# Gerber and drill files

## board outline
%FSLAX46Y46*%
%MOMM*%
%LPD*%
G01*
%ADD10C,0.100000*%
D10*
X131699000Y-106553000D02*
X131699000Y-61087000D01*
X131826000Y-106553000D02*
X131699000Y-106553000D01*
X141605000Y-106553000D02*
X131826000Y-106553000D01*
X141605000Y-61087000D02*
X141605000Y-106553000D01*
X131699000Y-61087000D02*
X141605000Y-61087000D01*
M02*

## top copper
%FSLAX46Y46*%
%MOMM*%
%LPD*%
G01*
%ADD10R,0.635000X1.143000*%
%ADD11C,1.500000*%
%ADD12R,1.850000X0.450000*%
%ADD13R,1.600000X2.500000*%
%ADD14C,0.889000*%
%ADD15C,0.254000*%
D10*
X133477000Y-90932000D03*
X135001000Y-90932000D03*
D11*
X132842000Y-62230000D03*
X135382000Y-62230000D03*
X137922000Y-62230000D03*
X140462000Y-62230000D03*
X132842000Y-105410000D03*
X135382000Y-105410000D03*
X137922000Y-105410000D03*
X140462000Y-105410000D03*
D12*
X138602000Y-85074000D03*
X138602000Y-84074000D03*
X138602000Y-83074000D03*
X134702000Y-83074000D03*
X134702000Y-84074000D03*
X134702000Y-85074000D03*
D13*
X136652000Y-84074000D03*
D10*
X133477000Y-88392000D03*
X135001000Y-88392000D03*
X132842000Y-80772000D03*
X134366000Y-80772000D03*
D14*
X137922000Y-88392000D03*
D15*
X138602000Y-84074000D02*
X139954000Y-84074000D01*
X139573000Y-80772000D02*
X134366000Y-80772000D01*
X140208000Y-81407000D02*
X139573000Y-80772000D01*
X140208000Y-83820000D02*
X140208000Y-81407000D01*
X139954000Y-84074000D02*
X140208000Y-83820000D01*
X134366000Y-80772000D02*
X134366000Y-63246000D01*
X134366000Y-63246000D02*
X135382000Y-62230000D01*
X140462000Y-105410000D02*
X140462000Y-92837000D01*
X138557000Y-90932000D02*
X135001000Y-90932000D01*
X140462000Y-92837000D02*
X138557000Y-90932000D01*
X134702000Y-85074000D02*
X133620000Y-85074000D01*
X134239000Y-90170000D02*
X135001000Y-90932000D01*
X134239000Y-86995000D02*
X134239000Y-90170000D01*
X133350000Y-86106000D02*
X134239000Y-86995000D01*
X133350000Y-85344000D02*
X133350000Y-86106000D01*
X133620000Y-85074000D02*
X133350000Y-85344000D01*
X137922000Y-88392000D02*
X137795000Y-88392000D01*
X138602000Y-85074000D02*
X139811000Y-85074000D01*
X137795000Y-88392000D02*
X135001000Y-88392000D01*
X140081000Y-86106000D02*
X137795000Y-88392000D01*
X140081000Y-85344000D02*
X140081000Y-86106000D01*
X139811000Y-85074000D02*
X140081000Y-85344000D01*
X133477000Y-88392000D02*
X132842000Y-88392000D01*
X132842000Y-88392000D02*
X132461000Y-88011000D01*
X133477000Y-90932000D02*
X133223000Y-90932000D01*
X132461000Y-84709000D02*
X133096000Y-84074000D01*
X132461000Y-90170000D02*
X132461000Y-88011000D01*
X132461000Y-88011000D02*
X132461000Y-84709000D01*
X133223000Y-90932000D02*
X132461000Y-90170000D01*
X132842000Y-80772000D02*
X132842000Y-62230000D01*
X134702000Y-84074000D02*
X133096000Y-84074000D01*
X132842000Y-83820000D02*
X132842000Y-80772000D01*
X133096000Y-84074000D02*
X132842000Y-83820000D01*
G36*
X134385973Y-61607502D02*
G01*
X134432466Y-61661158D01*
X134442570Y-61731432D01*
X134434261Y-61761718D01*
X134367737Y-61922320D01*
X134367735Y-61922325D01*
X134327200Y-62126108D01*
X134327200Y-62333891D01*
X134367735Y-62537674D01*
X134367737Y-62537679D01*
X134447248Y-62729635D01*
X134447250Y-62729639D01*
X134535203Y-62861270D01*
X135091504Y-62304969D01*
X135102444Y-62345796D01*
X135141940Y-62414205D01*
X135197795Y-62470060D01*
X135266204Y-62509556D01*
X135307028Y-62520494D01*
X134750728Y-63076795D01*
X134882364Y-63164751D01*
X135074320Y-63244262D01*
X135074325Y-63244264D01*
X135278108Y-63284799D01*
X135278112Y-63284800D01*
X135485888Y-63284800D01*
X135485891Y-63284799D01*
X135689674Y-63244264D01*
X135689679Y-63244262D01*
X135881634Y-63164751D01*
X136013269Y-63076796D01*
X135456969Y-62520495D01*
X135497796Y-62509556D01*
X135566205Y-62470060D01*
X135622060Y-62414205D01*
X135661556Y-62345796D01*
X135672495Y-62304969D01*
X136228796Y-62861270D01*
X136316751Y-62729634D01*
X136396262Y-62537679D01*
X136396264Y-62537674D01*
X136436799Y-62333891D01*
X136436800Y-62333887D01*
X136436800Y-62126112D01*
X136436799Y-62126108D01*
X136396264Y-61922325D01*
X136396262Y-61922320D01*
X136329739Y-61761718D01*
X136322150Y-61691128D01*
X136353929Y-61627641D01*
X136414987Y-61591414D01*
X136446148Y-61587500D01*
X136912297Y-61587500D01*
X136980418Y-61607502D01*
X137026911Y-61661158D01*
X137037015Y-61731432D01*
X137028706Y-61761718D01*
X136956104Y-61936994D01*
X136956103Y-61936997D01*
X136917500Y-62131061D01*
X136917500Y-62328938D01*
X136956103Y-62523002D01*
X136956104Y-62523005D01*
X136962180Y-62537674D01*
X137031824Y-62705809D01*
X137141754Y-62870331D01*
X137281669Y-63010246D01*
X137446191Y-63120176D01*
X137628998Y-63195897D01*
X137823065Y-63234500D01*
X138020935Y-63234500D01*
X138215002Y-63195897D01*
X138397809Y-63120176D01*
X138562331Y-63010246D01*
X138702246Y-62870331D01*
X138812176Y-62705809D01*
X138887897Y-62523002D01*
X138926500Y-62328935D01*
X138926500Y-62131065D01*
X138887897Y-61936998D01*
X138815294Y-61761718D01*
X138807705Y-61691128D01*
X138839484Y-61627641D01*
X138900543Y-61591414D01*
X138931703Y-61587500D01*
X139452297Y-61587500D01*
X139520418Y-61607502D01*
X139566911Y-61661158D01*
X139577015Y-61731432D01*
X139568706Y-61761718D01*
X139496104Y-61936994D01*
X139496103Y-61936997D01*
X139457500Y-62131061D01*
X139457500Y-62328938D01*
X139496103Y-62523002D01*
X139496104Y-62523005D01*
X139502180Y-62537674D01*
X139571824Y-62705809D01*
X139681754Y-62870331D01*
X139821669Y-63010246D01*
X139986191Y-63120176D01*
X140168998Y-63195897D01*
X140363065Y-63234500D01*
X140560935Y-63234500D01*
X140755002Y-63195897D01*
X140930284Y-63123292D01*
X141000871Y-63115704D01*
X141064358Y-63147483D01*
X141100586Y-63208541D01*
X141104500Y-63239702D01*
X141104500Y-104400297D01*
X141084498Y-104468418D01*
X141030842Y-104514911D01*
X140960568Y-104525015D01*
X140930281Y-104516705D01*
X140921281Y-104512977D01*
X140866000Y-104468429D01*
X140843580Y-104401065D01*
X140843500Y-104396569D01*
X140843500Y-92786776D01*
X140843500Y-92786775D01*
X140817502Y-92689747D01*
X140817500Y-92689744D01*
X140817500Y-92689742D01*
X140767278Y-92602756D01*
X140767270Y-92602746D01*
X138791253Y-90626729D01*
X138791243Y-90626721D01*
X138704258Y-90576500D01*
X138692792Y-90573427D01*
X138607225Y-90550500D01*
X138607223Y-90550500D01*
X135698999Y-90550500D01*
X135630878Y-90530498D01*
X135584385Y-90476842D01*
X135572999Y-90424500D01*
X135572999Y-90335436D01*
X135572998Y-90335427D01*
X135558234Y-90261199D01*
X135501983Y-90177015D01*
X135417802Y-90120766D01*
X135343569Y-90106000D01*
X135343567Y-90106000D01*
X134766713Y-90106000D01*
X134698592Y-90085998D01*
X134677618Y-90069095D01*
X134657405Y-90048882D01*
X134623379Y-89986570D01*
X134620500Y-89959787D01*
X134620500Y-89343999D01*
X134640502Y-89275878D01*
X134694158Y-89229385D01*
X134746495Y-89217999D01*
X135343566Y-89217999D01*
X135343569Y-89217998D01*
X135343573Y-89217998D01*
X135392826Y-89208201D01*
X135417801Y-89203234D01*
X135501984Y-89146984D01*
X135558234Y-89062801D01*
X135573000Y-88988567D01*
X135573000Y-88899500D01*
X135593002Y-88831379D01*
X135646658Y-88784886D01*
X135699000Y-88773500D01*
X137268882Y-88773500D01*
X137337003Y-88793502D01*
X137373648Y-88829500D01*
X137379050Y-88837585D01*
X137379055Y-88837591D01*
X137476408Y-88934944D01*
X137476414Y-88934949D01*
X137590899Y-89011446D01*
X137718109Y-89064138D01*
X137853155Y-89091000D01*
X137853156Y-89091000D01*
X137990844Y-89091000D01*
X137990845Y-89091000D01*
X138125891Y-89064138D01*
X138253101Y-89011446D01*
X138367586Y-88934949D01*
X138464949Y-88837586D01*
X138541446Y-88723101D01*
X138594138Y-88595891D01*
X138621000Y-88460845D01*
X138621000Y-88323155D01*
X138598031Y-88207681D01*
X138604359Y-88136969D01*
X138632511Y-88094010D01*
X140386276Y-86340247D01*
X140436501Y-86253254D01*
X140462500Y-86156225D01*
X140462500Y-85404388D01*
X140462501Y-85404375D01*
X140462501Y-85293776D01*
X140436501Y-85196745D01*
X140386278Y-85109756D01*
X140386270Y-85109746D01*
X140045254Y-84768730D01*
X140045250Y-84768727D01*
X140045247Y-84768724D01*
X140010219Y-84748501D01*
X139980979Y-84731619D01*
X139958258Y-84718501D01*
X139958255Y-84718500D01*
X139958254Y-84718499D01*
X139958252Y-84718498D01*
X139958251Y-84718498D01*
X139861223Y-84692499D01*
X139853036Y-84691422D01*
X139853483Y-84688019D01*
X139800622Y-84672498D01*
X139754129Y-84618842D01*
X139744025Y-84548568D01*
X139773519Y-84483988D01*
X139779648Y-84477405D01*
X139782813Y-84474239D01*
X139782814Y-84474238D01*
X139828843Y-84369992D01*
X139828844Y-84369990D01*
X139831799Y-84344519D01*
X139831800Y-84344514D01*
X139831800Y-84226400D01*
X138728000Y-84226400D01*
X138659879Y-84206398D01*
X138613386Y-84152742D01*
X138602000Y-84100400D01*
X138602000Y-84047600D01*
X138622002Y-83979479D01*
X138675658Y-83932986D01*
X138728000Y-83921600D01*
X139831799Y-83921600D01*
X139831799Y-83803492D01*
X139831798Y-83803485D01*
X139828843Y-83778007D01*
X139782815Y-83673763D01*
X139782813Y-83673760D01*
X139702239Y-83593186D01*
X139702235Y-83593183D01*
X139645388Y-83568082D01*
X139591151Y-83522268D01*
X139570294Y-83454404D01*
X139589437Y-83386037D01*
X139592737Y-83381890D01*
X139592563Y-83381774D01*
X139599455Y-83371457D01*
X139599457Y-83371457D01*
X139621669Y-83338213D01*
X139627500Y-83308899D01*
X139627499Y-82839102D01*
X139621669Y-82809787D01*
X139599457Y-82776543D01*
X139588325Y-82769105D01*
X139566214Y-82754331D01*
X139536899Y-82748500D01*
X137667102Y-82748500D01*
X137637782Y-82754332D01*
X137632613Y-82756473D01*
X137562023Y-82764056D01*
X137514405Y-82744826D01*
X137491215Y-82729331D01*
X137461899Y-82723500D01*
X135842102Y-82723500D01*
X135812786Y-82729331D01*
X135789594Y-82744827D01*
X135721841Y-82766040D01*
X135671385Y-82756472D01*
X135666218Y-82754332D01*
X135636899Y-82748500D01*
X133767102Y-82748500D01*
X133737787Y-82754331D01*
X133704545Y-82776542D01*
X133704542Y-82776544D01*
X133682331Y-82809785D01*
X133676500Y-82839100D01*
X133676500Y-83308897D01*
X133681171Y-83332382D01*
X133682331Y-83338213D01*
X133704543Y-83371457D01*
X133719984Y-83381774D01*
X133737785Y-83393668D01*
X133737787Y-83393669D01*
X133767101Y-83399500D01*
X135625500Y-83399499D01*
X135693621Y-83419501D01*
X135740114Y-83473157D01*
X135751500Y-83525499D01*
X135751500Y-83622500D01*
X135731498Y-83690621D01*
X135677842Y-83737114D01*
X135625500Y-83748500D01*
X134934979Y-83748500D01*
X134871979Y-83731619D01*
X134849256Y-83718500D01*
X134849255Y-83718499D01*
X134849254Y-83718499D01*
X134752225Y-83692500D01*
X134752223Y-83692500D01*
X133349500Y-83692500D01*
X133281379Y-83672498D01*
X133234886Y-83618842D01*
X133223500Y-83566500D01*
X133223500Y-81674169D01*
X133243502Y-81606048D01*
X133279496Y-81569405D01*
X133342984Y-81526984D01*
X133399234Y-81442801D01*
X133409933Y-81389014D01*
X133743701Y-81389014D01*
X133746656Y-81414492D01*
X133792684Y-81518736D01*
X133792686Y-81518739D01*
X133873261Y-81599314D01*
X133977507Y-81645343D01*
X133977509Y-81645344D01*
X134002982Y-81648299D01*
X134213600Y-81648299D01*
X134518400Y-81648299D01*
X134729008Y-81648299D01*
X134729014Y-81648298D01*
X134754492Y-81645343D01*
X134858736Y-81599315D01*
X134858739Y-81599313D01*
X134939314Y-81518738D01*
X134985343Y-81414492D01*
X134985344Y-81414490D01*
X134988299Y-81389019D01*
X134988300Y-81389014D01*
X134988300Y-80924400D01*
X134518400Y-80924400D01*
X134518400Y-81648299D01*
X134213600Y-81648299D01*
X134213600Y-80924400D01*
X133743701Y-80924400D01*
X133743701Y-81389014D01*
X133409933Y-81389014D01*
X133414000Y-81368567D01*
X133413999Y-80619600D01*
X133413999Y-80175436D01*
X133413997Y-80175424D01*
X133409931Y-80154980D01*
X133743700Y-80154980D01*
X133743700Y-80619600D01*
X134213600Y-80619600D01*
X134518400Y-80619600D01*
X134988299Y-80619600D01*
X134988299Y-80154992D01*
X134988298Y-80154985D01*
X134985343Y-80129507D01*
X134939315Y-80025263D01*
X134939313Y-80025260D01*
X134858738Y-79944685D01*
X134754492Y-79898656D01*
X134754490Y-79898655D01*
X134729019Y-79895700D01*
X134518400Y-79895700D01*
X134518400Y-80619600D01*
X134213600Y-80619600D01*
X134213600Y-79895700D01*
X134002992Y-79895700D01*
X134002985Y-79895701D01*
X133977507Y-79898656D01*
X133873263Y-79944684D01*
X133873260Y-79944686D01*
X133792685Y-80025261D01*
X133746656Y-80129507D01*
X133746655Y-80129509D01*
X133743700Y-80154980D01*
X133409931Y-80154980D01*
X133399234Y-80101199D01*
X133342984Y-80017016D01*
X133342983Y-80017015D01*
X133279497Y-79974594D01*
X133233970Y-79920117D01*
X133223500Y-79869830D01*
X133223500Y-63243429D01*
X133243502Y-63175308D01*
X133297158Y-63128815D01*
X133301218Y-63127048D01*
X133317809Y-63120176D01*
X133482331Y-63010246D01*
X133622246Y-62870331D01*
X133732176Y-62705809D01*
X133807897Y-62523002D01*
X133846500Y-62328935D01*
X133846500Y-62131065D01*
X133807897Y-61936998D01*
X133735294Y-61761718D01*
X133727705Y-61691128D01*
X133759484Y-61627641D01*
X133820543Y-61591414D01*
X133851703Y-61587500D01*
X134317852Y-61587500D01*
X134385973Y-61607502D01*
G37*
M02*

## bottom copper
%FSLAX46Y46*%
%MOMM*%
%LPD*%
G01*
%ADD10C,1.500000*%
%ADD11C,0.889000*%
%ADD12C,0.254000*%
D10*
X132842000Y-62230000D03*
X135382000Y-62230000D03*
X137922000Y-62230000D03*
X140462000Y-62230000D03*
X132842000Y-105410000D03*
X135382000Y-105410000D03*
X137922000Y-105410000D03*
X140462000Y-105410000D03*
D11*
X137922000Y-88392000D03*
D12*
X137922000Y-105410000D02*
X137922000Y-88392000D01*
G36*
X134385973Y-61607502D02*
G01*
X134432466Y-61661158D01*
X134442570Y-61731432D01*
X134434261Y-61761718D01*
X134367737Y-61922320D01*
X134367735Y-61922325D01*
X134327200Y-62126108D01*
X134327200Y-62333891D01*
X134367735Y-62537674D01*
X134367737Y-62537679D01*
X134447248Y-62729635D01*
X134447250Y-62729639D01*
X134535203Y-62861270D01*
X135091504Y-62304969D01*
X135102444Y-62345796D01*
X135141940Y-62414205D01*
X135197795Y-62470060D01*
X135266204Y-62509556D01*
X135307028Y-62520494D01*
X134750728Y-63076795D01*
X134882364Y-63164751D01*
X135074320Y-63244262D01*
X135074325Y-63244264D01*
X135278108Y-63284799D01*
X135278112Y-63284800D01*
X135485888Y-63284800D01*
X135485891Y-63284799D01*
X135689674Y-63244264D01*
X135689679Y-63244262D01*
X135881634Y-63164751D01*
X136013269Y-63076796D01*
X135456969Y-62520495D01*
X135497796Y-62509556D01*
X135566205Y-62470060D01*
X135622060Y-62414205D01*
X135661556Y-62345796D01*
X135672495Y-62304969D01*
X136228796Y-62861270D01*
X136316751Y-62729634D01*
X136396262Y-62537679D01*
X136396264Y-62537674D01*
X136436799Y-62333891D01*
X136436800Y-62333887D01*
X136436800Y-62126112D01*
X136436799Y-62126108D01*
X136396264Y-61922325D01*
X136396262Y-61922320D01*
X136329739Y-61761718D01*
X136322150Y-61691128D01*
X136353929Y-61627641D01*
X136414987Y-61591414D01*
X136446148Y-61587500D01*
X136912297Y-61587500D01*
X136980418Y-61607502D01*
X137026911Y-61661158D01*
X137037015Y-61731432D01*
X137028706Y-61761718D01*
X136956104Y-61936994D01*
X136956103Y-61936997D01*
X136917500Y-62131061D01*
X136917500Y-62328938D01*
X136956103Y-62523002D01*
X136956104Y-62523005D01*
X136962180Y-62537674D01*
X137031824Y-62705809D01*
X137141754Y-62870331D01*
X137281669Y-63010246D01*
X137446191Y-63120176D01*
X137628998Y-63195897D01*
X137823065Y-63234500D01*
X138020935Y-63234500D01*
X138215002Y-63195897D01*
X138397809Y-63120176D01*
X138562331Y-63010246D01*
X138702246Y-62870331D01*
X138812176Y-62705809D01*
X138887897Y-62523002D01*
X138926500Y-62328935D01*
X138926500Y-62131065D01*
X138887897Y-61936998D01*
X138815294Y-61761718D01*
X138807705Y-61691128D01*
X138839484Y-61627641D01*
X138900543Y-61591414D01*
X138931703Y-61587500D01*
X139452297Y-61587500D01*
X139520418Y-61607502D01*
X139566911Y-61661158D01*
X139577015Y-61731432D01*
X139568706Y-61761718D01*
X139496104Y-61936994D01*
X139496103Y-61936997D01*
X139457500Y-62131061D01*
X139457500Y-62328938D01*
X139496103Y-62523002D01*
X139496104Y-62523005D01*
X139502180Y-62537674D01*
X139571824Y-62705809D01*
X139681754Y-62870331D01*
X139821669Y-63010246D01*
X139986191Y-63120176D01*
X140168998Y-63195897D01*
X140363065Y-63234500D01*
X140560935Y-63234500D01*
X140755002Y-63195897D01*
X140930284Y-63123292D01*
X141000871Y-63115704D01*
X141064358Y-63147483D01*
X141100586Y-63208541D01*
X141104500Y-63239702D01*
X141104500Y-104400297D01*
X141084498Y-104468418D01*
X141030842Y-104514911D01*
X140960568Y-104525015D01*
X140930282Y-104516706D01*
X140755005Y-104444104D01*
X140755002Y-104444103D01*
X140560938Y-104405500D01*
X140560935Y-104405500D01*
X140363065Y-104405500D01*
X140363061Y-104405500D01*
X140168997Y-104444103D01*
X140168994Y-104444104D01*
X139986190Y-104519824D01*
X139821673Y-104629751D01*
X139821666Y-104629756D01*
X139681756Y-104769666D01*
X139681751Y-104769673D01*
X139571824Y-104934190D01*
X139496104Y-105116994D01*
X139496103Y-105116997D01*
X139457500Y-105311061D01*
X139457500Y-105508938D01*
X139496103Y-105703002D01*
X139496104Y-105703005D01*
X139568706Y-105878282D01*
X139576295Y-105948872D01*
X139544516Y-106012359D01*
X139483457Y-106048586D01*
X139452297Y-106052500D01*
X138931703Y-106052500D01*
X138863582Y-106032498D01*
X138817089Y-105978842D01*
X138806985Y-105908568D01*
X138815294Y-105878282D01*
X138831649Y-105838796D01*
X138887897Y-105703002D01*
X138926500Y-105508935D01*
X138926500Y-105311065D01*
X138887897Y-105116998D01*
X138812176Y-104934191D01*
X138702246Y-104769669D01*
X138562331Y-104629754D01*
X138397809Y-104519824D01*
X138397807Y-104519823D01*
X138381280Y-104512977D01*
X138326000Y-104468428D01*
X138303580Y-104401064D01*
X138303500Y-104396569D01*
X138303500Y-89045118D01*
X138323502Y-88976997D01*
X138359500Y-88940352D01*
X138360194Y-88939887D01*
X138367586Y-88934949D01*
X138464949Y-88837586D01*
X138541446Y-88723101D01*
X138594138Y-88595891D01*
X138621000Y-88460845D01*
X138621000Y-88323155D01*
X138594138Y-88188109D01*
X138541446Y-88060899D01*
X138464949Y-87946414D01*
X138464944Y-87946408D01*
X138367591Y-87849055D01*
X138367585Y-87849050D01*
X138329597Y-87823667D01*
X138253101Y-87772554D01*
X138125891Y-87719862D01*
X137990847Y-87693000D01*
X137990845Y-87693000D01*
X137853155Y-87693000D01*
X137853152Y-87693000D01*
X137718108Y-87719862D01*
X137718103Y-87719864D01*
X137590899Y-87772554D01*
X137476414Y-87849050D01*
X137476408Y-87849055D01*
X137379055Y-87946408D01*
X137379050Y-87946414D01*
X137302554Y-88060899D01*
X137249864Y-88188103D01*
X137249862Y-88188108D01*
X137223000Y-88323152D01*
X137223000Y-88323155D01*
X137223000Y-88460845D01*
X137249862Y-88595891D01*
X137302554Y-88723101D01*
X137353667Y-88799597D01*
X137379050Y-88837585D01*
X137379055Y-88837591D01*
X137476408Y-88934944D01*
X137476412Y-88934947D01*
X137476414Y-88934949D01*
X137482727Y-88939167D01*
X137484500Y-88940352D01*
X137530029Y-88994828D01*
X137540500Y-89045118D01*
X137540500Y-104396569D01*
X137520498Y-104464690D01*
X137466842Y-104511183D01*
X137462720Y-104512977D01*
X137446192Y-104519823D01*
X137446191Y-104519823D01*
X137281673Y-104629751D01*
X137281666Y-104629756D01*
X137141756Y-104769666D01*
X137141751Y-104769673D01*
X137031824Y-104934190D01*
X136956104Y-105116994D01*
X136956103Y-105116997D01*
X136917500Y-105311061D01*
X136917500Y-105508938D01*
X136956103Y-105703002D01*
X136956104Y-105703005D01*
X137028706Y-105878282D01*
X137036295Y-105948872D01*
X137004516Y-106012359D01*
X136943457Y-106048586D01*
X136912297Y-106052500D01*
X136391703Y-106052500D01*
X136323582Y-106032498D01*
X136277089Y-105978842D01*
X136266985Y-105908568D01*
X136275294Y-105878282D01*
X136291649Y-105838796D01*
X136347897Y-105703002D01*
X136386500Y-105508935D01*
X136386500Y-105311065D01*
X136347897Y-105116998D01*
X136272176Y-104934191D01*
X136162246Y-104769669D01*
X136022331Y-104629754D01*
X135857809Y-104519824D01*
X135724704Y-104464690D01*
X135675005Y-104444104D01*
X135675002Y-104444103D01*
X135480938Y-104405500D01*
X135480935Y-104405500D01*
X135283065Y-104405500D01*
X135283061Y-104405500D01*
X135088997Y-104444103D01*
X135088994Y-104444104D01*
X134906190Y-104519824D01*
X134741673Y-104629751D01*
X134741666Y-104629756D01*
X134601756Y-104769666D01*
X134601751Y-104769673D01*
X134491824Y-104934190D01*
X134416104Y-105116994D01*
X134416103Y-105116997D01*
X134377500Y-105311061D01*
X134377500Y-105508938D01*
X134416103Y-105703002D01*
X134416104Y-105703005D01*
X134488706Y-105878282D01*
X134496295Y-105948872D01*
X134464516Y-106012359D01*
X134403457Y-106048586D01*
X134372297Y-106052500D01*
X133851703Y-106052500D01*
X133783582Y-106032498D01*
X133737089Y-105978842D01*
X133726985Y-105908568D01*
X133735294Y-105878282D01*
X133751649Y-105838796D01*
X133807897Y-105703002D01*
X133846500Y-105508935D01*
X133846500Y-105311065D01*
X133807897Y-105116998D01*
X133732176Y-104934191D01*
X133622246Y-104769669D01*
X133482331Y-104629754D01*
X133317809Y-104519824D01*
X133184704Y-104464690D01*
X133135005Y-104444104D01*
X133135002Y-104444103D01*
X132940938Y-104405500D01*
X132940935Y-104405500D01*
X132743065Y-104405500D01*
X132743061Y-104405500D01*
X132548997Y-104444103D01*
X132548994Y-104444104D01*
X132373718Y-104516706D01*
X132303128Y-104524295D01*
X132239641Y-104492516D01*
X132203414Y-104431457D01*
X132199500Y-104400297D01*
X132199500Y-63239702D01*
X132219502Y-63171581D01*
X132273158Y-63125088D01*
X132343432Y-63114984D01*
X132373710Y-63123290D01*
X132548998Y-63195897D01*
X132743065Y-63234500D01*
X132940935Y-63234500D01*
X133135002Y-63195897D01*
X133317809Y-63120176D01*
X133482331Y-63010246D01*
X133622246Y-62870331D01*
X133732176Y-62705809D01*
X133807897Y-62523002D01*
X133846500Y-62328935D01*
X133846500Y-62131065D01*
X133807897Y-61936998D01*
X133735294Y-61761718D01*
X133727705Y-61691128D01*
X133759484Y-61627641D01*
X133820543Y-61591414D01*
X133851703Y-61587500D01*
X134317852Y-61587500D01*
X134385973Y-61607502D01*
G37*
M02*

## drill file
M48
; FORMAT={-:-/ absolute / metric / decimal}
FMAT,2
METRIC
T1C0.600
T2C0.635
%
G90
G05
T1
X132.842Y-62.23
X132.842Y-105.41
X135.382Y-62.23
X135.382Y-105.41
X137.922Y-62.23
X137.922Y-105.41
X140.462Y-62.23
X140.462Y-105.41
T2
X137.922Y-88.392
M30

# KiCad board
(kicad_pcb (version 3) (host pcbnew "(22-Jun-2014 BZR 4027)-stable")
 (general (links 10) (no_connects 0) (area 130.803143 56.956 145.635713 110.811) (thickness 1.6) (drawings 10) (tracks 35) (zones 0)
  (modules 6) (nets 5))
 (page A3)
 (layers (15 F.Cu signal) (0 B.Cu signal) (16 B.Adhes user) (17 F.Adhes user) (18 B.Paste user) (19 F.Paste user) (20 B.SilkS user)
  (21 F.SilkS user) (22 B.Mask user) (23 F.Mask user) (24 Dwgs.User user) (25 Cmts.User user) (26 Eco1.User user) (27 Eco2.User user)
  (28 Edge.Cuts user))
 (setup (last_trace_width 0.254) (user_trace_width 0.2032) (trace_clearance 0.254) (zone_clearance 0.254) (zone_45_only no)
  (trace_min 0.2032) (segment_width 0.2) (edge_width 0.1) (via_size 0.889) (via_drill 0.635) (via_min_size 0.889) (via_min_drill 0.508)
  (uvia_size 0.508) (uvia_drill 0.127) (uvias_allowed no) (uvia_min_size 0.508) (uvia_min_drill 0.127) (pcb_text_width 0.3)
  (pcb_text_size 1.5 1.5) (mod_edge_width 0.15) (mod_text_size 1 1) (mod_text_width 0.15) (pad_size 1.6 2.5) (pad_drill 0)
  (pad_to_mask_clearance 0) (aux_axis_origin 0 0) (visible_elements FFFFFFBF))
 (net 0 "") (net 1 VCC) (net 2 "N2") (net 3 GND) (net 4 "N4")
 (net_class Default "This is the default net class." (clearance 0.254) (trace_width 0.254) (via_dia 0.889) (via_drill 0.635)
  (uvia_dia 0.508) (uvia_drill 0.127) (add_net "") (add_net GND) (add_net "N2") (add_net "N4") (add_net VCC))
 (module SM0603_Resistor (layer F.Cu) (at 134.239 90.932)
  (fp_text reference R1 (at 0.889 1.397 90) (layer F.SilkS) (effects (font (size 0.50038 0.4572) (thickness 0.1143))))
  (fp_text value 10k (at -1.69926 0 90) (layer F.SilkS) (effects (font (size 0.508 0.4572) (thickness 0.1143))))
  (pad 1 smd rect (at -0.762 0) (size 0.635 1.143) (layers F.Cu F.Paste F.Mask) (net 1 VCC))
  (pad 2 smd rect (at 0.762 0) (size 0.635 1.143) (layers F.Cu F.Paste F.Mask) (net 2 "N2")))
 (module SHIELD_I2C (layer F.Cu) (at 136.652 83.82)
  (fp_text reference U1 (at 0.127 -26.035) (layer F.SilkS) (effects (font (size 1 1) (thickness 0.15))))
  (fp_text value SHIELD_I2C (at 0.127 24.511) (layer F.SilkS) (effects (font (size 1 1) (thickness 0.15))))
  (pad 1 thru_hole circle (at -3.81 -21.59) (size 1.5 1.5) (drill 0.6) (layers *.Cu *.Mask F.SilkS) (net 1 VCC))
  (pad 2 thru_hole circle (at -1.27 -21.59) (size 1.5 1.5) (drill 0.6) (layers *.Cu *.Mask F.SilkS) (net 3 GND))
  (pad 3 thru_hole circle (at 1.27 -21.59) (size 1.5 1.5) (drill 0.6) (layers *.Cu *.Mask F.SilkS))
  (pad 4 thru_hole circle (at 3.81 -21.59) (size 1.5 1.5) (drill 0.6) (layers *.Cu *.Mask F.SilkS))
  (pad 5 thru_hole circle (at -3.81 21.59) (size 1.5 1.5) (drill 0.6) (layers *.Cu *.Mask F.SilkS))
  (pad 6 thru_hole circle (at -1.27 21.59) (size 1.5 1.5) (drill 0.6) (layers *.Cu *.Mask F.SilkS))
  (pad 7 thru_hole circle (at 1.27 21.59) (size 1.5 1.5) (drill 0.6) (layers *.Cu *.Mask F.SilkS) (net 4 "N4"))
  (pad 8 thru_hole circle (at 3.81 21.59) (size 1.5 1.5) (drill 0.6) (layers *.Cu *.Mask F.SilkS) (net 2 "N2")))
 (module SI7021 (layer F.Cu) (at 136.652 84.074 180) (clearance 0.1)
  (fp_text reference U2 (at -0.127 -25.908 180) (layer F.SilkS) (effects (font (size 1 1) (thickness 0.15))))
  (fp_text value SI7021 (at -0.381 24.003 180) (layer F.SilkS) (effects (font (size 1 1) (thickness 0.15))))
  (pad 1 smd rect (at -1.95 -1 180) (size 1.85 0.45) (layers F.Cu F.Paste F.Mask) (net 4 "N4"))
  (pad 2 smd rect (at -1.95 0 180) (size 1.85 0.45) (layers F.Cu F.Paste F.Mask) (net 3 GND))
  (pad 3 smd rect (at -1.95 1 180) (size 1.85 0.45) (layers F.Cu F.Paste F.Mask))
  (pad 4 smd rect (at 1.95 1 180) (size 1.85 0.45) (layers F.Cu F.Paste F.Mask))
  (pad 5 smd rect (at 1.95 0 180) (size 1.85 0.45) (layers F.Cu F.Paste F.Mask) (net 1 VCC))
  (pad 6 smd rect (at 1.95 -1 180) (size 1.85 0.45) (layers F.Cu F.Paste F.Mask) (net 2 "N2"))
  (pad 7 smd rect (at 0 0 180) (size 1.6 2.5) (layers F.Cu F.Paste F.Mask)))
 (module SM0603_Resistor (layer F.Cu) (at 134.239 88.392)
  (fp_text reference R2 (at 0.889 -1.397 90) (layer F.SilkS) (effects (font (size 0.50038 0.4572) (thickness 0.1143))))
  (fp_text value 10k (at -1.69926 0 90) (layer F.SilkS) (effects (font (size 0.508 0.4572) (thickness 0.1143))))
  (pad 1 smd rect (at -0.762 0) (size 0.635 1.143) (layers F.Cu F.Paste F.Mask) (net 1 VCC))
  (pad 2 smd rect (at 0.762 0) (size 0.635 1.143) (layers F.Cu F.Paste F.Mask) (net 4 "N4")))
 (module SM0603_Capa (layer F.Cu) (at 133.604 80.772)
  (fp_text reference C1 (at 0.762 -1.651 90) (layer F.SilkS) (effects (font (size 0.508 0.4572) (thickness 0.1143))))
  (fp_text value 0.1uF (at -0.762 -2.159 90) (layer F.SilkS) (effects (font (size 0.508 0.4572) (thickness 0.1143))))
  (pad 1 smd rect (at -0.762 0) (size 0.635 1.143) (layers F.Cu F.Paste F.Mask) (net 1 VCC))
  (pad 2 smd rect (at 0.762 0) (size 0.635 1.143) (layers F.Cu F.Paste F.Mask) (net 3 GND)))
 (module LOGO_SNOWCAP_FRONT (layer F.Cu) (at 138.811 71.501 90)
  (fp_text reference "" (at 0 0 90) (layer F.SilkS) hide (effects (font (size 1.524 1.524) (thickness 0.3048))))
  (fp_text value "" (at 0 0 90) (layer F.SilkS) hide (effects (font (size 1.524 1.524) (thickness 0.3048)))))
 (gr_line (start 131.699 106.553) (end 131.699 61.087) (angle 90) (layer Edge.Cuts) (width 0.1))
 (gr_line (start 131.826 106.553) (end 131.699 106.553) (angle 90) (layer Edge.Cuts) (width 0.1))
 (gr_line (start 141.605 106.553) (end 131.826 106.553) (angle 90) (layer Edge.Cuts) (width 0.1))
 (gr_line (start 141.605 61.087) (end 141.605 106.553) (angle 90) (layer Edge.Cuts) (width 0.1))
 (gr_line (start 131.699 61.087) (end 141.605 61.087) (angle 90) (layer Edge.Cuts) (width 0.1))
 (segment (start 138.602 84.074) (end 139.954 84.074) (width 0.254) (layer F.Cu) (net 3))
 (segment (start 139.573 80.772) (end 134.366 80.772) (width 0.254) (layer F.Cu) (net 3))
 (segment (start 140.208 81.407) (end 139.573 80.772) (width 0.254) (layer F.Cu) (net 3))
 (segment (start 140.208 83.82) (end 140.208 81.407) (width 0.254) (layer F.Cu) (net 3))
 (segment (start 139.954 84.074) (end 140.208 83.82) (width 0.254) (layer F.Cu) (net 3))
 (segment (start 134.366 80.772) (end 134.366 63.246) (width 0.254) (layer F.Cu) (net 3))
 (segment (start 134.366 63.246) (end 135.382 62.23) (width 0.254) (layer F.Cu) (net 3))
 (segment (start 140.462 105.41) (end 140.462 92.837) (width 0.254) (layer F.Cu) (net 2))
 (segment (start 138.557 90.932) (end 135.001 90.932) (width 0.254) (layer F.Cu) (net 2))
 (segment (start 140.462 92.837) (end 138.557 90.932) (width 0.254) (layer F.Cu) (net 2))
 (segment (start 134.702 85.074) (end 133.62 85.074) (width 0.254) (layer F.Cu) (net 2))
 (segment (start 134.239 90.17) (end 135.001 90.932) (width 0.254) (layer F.Cu) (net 2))
 (segment (start 134.239 86.995) (end 134.239 90.17) (width 0.254) (layer F.Cu) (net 2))
 (segment (start 133.35 86.106) (end 134.239 86.995) (width 0.254) (layer F.Cu) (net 2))
 (segment (start 133.35 85.344) (end 133.35 86.106) (width 0.254) (layer F.Cu) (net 2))
 (segment (start 133.62 85.074) (end 133.35 85.344) (width 0.254) (layer F.Cu) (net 2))
 (segment (start 137.922 105.41) (end 137.922 88.392) (width 0.254) (layer B.Cu) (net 4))
 (segment (start 137.922 88.392) (end 137.795 88.392) (width 0.254) (layer F.Cu) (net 4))
 (via (at 137.922 88.392) (size 0.889) (layers F.Cu B.Cu) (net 4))
 (segment (start 138.602 85.074) (end 139.811 85.074) (width 0.254) (layer F.Cu) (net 4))
 (segment (start 137.795 88.392) (end 135.001 88.392) (width 0.254) (layer F.Cu) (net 4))
 (segment (start 140.081 86.106) (end 137.795 88.392) (width 0.254) (layer F.Cu) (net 4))
 (segment (start 140.081 85.344) (end 140.081 86.106) (width 0.254) (layer F.Cu) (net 4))
 (segment (start 139.811 85.074) (end 140.081 85.344) (width 0.254) (layer F.Cu) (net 4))
 (segment (start 133.477 88.392) (end 132.842 88.392) (width 0.254) (layer F.Cu) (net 1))
 (segment (start 132.842 88.392) (end 132.461 88.011) (width 0.254) (layer F.Cu) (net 1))
 (segment (start 133.477 90.932) (end 133.223 90.932) (width 0.254) (layer F.Cu) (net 1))
 (segment (start 132.461 84.709) (end 133.096 84.074) (width 0.254) (layer F.Cu) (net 1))
 (segment (start 132.461 90.17) (end 132.461 88.011) (width 0.254) (layer F.Cu) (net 1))
 (segment (start 132.461 88.011) (end 132.461 84.709) (width 0.254) (layer F.Cu) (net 1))
 (segment (start 133.223 90.932) (end 132.461 90.17) (width 0.254) (layer F.Cu) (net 1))
 (segment (start 132.842 80.772) (end 132.842 62.23) (width 0.254) (layer F.Cu) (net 1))
 (segment (start 134.702 84.074) (end 133.096 84.074) (width 0.254) (layer F.Cu) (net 1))
 (segment (start 132.842 83.82) (end 132.842 80.772) (width 0.254) (layer F.Cu) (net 1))
 (segment (start 133.096 84.074) (end 132.842 83.82) (width 0.254) (layer F.Cu) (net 1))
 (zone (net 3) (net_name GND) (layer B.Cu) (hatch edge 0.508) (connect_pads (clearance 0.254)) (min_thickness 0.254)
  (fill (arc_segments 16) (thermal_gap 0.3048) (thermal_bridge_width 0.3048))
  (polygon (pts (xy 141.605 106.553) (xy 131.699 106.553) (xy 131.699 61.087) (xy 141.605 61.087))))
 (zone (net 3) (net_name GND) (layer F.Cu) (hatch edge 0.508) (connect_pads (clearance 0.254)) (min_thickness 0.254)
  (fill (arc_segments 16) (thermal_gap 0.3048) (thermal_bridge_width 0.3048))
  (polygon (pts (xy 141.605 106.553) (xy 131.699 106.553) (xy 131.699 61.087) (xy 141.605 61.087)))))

